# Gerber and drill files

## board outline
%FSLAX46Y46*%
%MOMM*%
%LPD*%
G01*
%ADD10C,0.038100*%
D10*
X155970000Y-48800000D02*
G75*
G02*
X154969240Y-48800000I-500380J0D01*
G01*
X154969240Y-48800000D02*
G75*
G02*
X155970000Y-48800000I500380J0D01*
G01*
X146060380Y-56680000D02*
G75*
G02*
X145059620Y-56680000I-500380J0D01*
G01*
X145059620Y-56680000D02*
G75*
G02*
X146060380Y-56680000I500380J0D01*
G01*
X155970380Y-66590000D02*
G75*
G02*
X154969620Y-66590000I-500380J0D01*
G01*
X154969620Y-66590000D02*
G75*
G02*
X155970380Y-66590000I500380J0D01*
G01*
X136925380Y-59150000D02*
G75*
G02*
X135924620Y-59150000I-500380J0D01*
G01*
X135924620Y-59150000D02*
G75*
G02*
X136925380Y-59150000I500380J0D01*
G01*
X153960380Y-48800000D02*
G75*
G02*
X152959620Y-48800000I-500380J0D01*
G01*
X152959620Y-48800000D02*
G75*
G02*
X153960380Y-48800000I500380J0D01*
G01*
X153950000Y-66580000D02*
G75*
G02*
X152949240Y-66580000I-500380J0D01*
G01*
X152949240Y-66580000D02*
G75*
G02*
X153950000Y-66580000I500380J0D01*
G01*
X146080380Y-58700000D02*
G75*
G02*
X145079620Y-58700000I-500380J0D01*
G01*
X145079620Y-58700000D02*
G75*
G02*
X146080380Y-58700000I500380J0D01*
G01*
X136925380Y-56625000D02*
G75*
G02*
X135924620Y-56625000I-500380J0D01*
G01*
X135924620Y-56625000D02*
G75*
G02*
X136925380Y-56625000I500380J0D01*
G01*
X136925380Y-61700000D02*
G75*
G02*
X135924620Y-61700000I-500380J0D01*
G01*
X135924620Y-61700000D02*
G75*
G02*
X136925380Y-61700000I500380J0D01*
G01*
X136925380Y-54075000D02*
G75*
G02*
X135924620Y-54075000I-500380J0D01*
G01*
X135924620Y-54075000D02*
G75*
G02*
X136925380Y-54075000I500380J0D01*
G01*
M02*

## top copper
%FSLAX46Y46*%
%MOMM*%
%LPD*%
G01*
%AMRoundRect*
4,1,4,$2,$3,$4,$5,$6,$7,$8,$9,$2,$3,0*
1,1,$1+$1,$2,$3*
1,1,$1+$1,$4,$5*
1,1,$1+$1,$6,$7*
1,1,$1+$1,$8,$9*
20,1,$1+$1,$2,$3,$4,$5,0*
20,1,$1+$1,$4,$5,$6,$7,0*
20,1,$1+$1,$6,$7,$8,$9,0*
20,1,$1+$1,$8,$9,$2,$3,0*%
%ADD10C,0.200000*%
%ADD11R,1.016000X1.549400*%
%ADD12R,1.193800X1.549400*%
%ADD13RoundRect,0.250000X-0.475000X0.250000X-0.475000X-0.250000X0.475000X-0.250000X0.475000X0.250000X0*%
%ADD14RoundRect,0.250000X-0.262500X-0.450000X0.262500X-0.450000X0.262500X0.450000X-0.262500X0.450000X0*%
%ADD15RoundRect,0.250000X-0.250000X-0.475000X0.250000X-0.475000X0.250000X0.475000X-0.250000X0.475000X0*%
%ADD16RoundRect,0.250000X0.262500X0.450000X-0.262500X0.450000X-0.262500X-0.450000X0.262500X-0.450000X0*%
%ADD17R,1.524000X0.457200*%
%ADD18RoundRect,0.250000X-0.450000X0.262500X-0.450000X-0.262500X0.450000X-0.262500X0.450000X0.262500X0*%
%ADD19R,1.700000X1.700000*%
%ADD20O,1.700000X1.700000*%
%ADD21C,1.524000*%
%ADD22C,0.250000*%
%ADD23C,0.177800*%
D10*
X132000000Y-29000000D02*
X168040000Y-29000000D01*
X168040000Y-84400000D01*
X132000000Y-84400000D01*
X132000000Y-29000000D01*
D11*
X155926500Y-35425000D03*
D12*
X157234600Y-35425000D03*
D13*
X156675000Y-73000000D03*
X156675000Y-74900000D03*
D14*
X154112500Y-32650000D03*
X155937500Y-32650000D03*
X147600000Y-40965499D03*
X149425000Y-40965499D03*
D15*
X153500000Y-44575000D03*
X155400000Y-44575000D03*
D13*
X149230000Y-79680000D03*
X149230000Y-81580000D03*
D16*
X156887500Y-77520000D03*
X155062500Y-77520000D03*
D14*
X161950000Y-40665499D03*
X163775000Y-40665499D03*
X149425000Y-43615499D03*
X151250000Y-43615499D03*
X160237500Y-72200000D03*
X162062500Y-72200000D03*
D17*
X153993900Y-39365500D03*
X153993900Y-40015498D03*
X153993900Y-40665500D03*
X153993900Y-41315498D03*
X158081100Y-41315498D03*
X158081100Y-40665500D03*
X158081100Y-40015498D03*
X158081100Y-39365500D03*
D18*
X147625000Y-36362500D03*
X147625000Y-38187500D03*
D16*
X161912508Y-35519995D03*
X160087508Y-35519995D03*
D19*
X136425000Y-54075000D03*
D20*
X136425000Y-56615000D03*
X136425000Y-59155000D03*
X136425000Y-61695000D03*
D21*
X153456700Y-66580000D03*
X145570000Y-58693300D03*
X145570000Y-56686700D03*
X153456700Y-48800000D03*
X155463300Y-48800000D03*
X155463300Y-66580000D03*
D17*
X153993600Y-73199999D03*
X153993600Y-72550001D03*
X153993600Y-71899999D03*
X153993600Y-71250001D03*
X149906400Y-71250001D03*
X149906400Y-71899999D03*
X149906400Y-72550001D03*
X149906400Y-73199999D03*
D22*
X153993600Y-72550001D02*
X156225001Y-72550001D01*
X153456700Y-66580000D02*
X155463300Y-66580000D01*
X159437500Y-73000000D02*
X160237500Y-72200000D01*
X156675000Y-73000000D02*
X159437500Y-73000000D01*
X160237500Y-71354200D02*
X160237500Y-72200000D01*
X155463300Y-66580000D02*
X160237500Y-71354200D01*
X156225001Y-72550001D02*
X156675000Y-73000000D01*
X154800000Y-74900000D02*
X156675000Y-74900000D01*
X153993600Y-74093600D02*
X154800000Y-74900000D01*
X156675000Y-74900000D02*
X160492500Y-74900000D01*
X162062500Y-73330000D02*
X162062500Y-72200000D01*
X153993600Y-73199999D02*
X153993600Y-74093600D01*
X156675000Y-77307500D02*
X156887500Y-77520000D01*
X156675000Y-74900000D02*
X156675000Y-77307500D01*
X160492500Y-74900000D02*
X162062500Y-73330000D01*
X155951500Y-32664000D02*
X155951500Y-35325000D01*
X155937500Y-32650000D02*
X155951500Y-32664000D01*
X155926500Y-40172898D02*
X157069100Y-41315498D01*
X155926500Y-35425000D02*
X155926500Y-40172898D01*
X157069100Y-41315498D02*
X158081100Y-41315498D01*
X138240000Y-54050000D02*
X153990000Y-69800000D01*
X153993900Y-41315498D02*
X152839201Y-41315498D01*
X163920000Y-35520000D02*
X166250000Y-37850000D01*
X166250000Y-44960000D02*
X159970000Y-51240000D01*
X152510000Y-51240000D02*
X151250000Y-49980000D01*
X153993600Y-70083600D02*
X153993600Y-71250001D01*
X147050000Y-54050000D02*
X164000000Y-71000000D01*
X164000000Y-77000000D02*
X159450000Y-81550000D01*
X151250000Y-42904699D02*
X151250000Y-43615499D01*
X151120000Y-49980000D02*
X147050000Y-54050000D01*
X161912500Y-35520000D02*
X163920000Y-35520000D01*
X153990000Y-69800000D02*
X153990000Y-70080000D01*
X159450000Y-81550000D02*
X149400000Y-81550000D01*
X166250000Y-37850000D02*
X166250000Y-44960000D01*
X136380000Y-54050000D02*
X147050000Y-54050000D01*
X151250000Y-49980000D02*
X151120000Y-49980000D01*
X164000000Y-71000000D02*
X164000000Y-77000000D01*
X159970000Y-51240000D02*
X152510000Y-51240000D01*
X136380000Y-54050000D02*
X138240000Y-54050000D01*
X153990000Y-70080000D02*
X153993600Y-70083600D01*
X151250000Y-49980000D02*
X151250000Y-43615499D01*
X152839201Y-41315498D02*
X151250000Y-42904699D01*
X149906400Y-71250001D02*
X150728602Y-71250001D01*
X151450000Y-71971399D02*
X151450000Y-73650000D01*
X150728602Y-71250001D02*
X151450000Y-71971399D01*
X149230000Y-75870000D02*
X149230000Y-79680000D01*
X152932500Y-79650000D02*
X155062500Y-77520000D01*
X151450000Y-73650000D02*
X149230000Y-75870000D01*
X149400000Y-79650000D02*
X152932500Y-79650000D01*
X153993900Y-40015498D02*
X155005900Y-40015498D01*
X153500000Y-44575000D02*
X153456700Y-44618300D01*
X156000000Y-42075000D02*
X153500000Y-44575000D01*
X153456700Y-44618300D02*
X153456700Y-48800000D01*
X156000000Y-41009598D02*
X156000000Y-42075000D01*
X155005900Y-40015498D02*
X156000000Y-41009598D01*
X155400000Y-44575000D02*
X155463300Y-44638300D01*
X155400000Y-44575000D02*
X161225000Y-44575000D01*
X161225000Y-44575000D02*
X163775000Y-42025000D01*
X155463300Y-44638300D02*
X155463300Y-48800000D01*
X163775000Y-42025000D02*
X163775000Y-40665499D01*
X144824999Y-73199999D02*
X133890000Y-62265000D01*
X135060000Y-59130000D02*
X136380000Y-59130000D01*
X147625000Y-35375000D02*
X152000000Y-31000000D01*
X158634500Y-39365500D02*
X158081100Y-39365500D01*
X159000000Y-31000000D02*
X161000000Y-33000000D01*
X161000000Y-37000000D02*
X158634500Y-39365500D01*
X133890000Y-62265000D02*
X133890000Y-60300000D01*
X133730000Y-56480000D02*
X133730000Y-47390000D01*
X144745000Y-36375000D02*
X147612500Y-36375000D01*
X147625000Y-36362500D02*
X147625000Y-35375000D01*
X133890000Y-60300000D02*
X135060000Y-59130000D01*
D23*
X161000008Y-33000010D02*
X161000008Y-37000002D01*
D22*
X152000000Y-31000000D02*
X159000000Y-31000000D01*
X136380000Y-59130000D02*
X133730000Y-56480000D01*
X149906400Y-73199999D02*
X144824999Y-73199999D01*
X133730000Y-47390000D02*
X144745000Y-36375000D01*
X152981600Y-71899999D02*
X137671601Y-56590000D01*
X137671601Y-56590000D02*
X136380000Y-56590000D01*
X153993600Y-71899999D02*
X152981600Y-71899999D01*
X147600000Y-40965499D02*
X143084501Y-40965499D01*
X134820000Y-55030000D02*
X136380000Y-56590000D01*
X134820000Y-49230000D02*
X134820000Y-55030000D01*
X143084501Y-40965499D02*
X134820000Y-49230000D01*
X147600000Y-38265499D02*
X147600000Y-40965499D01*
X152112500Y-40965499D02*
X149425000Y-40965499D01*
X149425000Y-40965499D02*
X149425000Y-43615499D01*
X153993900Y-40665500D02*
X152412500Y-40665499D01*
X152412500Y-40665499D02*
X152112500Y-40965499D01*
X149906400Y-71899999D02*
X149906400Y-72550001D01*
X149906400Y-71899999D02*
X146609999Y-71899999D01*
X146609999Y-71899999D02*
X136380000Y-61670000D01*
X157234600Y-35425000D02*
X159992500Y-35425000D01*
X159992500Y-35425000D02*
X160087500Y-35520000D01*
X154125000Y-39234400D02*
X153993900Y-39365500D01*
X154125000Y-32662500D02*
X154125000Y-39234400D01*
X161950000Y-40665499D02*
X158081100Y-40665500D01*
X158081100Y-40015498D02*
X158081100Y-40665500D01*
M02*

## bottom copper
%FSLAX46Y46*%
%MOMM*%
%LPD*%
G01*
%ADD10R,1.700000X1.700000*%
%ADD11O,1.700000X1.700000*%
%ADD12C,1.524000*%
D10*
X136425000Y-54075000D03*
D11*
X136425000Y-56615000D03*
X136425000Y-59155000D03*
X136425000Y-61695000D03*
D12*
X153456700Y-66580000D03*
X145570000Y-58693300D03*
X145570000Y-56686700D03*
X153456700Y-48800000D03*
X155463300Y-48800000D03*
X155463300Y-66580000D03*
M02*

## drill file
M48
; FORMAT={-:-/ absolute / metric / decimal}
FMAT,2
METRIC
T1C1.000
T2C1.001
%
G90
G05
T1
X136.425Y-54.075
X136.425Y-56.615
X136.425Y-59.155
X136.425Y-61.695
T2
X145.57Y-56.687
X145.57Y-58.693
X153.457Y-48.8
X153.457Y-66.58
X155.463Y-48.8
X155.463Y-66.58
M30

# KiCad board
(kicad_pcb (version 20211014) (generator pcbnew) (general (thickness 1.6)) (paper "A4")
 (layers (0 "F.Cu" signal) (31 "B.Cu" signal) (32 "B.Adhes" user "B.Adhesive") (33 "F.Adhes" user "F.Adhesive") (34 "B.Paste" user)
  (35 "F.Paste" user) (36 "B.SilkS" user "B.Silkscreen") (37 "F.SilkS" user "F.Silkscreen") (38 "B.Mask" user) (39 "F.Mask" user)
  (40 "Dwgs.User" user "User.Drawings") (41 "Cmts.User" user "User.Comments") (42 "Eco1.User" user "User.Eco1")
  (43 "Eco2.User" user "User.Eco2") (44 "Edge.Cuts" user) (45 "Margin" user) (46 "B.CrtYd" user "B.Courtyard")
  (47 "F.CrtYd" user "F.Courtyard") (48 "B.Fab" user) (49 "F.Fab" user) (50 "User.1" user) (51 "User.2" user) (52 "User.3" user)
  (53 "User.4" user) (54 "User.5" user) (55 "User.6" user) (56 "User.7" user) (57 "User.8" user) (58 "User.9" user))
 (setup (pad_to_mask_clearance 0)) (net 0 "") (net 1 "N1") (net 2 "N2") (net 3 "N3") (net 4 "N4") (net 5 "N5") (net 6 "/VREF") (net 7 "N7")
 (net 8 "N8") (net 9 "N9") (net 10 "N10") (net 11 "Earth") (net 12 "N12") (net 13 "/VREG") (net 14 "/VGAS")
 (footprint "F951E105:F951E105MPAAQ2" (layer "F.Cu") (at 156.625 35.425)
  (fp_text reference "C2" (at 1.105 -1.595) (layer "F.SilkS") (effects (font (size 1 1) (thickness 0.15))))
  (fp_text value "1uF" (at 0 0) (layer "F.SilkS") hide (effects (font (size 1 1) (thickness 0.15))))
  (pad "1" smd rect (at -0.6985 0) (size 1.016 1.5494) (layers "F.Cu" "F.Paste" "F.Mask") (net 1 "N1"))
  (pad "2" smd rect (at 0.6096 0) (size 1.1938 1.5494) (layers "F.Cu" "F.Paste" "F.Mask") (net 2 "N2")))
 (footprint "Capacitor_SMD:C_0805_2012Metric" (layer "F.Cu") (at 156.675 73.95 -90)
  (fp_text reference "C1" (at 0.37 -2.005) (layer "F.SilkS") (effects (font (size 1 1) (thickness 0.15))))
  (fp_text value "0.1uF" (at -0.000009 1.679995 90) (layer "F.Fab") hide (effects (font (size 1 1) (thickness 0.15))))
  (pad "1" smd roundrect (at -0.95 0 270) (size 1 1.45) (layers "F.Cu" "F.Paste" "F.Mask") (roundrect_rratio 0.25) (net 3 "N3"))
  (pad "2" smd roundrect (at 0.95 0 270) (size 1 1.45) (layers "F.Cu" "F.Paste" "F.Mask") (roundrect_rratio 0.25) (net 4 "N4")))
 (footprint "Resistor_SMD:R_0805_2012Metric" (layer "F.Cu") (at 155.025 32.65)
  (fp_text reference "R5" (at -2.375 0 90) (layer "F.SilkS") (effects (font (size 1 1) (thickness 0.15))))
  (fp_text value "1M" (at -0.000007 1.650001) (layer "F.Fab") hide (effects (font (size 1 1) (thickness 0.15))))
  (pad "1" smd roundrect (at -0.9125 0) (size 1.025 1.4) (layers "F.Cu" "F.Paste" "F.Mask") (roundrect_rratio 0.243902439) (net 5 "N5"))
  (pad "2" smd roundrect (at 0.9125 0) (size 1.025 1.4) (layers "F.Cu" "F.Paste" "F.Mask") (roundrect_rratio 0.243902439) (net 1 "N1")))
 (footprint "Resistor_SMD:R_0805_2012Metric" (layer "F.Cu") (at 148.5125 40.965499)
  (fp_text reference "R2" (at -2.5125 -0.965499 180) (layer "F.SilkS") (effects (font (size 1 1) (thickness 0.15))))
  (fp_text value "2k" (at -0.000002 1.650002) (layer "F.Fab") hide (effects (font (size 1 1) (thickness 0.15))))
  (pad "1" smd roundrect (at -0.9125 0) (size 1.025 1.4) (layers "F.Cu" "F.Paste" "F.Mask") (roundrect_rratio 0.243902439) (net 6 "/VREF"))
  (pad "2" smd roundrect (at 0.9125 0) (size 1.025 1.4) (layers "F.Cu" "F.Paste" "F.Mask") (roundrect_rratio 0.243902439) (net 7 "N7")))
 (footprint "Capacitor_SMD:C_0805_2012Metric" (layer "F.Cu") (at 154.45 44.575)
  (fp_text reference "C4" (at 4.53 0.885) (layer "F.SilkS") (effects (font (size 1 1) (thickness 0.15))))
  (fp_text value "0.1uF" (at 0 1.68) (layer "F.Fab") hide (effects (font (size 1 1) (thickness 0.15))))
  (pad "1" smd roundrect (at -0.95 0) (size 1 1.45) (layers "F.Cu" "F.Paste" "F.Mask") (roundrect_rratio 0.25) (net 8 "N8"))
  (pad "2" smd roundrect (at 0.95 0) (size 1 1.45) (layers "F.Cu" "F.Paste" "F.Mask") (roundrect_rratio 0.25) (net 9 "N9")))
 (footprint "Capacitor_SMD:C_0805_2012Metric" (layer "F.Cu") (at 149.23 80.63 -90)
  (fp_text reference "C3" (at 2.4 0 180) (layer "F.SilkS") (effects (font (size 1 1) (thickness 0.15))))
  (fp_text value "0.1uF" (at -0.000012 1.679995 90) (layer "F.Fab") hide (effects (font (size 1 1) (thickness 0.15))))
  (pad "1" smd roundrect (at -0.95 0 270) (size 1 1.45) (layers "F.Cu" "F.Paste" "F.Mask") (roundrect_rratio 0.25) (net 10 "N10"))
  (pad "2" smd roundrect (at 0.95 0 270) (size 1 1.45) (layers "F.Cu" "F.Paste" "F.Mask") (roundrect_rratio 0.25) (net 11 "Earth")))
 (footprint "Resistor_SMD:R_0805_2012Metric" (layer "F.Cu") (at 155.975 77.52 180)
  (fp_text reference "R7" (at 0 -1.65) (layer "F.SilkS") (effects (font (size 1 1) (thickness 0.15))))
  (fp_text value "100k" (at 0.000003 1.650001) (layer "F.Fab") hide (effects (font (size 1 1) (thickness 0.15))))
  (pad "1" smd roundrect (at -0.9125 0 180) (size 1.025 1.4) (layers "F.Cu" "F.Paste" "F.Mask") (roundrect_rratio 0.243902439) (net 4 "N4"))
  (pad "2" smd roundrect (at 0.9125 0 180) (size 1.025 1.4) (layers "F.Cu" "F.Paste" "F.Mask") (roundrect_rratio 0.243902439) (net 10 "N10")))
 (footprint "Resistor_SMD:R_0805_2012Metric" (layer "F.Cu") (at 162.8625 40.665499)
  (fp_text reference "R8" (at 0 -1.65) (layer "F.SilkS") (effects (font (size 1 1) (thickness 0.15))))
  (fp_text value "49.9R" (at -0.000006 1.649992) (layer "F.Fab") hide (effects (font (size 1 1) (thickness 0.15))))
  (pad "1" smd roundrect (at -0.9125 0) (size 1.025 1.4) (layers "F.Cu" "F.Paste" "F.Mask") (roundrect_rratio 0.243902439) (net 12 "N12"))
  (pad "2" smd roundrect (at 0.9125 0) (size 1.025 1.4) (layers "F.Cu" "F.Paste" "F.Mask") (roundrect_rratio 0.243902439) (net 9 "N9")))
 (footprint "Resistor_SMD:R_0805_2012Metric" (layer "F.Cu") (at 150.3375 43.615499)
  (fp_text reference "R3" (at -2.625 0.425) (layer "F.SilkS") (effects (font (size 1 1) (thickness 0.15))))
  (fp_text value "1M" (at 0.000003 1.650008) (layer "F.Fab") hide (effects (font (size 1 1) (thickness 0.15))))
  (pad "1" smd roundrect (at -0.9125 0) (size 1.025 1.4) (layers "F.Cu" "F.Paste" "F.Mask") (roundrect_rratio 0.243902439) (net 7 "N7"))
  (pad "2" smd roundrect (at 0.9125 0) (size 1.025 1.4) (layers "F.Cu" "F.Paste" "F.Mask") (roundrect_rratio 0.243902439) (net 11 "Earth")))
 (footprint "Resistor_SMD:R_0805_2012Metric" (layer "F.Cu") (at 161.15 72.2)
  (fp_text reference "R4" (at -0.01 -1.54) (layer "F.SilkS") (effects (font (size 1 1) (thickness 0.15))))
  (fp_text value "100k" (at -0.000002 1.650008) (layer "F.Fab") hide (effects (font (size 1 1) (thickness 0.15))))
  (pad "1" smd roundrect (at -0.9125 0) (size 1.025 1.4) (layers "F.Cu" "F.Paste" "F.Mask") (roundrect_rratio 0.243902439) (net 3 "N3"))
  (pad "2" smd roundrect (at 0.9125 0) (size 1.025 1.4) (layers "F.Cu" "F.Paste" "F.Mask") (roundrect_rratio 0.243902439) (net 4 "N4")))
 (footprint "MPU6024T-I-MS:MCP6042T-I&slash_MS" (layer "F.Cu") (at 156.0375 40.340499)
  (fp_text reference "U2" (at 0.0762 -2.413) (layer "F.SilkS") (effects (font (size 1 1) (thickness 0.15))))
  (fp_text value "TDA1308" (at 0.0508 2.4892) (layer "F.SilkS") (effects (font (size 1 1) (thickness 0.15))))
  (pad "1" smd rect (at -2.0436 -0.974999) (size 1.524 0.4572) (layers "F.Cu" "F.Paste" "F.Mask") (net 5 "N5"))
  (pad "2" smd rect (at -2.0436 -0.325001) (size 1.524 0.4572) (layers "F.Cu" "F.Paste" "F.Mask") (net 8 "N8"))
  (pad "3" smd rect (at -2.0436 0.325001) (size 1.524 0.4572) (layers "F.Cu" "F.Paste" "F.Mask") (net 7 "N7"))
  (pad "4" smd rect (at -2.0436 0.974999) (size 1.524 0.4572) (layers "F.Cu" "F.Paste" "F.Mask") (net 11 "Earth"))
  (pad "5" smd rect (at 2.0436 0.974999) (size 1.524 0.4572) (layers "F.Cu" "F.Paste" "F.Mask") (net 1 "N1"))
  (pad "6" smd rect (at 2.0436 0.325001) (size 1.524 0.4572) (layers "F.Cu" "F.Paste" "F.Mask") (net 12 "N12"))
  (pad "7" smd rect (at 2.0436 -0.325001) (size 1.524 0.4572) (layers "F.Cu" "F.Paste" "F.Mask") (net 12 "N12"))
  (pad "8" smd rect (at 2.0436 -0.974999) (size 1.524 0.4572) (layers "F.Cu" "F.Paste" "F.Mask") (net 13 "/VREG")))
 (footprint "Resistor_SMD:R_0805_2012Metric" (layer "F.Cu") (at 147.625 37.275 -90)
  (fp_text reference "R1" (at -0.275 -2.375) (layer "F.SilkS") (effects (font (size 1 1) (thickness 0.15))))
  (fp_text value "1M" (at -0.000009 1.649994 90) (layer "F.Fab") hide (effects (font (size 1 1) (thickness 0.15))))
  (pad "1" smd roundrect (at -0.9125 0 270) (size 1.025 1.4) (layers "F.Cu" "F.Paste" "F.Mask") (roundrect_rratio 0.243902439)
   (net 13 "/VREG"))
  (pad "2" smd roundrect (at 0.9125 0 270) (size 1.025 1.4) (layers "F.Cu" "F.Paste" "F.Mask") (roundrect_rratio 0.243902439)
   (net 6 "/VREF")))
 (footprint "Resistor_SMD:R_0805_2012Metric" (layer "F.Cu") (at 161.000008 35.519995 180)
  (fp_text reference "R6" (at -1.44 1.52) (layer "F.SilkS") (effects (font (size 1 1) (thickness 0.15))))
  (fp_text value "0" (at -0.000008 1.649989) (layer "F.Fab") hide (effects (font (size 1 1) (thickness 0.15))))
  (pad "1" smd roundrect (at -0.9125 0 180) (size 1.025 1.4) (layers "F.Cu" "F.Paste" "F.Mask") (roundrect_rratio 0.243902439)
   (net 11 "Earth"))
  (pad "2" smd roundrect (at 0.9125 0 180) (size 1.025 1.4) (layers "F.Cu" "F.Paste" "F.Mask") (roundrect_rratio 0.243902439) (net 2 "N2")))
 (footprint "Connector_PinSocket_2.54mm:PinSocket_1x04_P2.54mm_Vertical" (layer "F.Cu") (at 136.425 54.075)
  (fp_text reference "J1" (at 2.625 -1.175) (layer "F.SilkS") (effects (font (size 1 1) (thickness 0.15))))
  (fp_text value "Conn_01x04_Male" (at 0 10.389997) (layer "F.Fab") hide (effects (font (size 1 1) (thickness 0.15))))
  (pad "1" thru_hole rect (at 0 0) (size 1.7 1.7) (drill 1) (layers *.Cu *.Mask) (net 11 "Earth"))
  (pad "2" thru_hole oval (at 0 2.54) (size 1.7 1.7) (drill 1) (layers *.Cu *.Mask) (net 6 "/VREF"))
  (pad "3" thru_hole oval (at 0 5.08) (size 1.7 1.7) (drill 1) (layers *.Cu *.Mask) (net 13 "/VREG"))
  (pad "4" thru_hole oval (at 0 7.62) (size 1.7 1.7) (drill 1) (layers *.Cu *.Mask) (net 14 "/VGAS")))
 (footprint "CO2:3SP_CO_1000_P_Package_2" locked (layer "F.Cu") (at 154.46 57.69)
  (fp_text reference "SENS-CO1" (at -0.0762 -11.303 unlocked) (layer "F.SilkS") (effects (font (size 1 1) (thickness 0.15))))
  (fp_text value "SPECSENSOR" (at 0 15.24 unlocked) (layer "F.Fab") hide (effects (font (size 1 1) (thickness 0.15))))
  (pad "1" thru_hole circle locked (at -1.0033 8.89) (size 1.524 1.524) (drill 1.00076) (layers *.Cu *.Mask) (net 3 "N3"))
  (pad "2" thru_hole circle locked (at -8.89 1.0033) (size 1.524 1.524) (drill 1.00076) (layers *.Cu *.Mask))
  (pad "3" thru_hole circle locked (at -8.89 -1.0033) (size 1.524 1.524) (drill 1.00076) (layers *.Cu *.Mask))
  (pad "4" thru_hole circle locked (at -1.0033 -8.89) (size 1.524 1.524) (drill 1.00076) (layers *.Cu *.Mask) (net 8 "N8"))
  (pad "5" thru_hole circle locked (at 1.0033 -8.89) (size 1.524 1.524) (drill 1.00076) (layers *.Cu *.Mask) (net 9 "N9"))
  (pad "6" thru_hole circle locked (at 1.0033 8.89) (size 1.524 1.524) (drill 1.00076) (layers *.Cu "F.Mask") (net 3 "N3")))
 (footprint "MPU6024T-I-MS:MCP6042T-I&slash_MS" (layer "F.Cu") (at 151.95 72.225 180)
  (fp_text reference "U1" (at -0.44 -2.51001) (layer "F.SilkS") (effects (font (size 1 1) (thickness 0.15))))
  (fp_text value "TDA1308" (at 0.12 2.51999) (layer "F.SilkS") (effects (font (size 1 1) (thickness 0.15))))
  (pad "1" smd rect (at -2.0436 -0.974999 180) (size 1.524 0.4572) (layers "F.Cu" "F.Paste" "F.Mask") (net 4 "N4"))
  (pad "2" smd rect (at -2.0436 -0.325001 180) (size 1.524 0.4572) (layers "F.Cu" "F.Paste" "F.Mask") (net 3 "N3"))
  (pad "3" smd rect (at -2.0436 0.325001 180) (size 1.524 0.4572) (layers "F.Cu" "F.Paste" "F.Mask") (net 6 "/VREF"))
  (pad "4" smd rect (at -2.0436 0.974999 180) (size 1.524 0.4572) (layers "F.Cu" "F.Paste" "F.Mask") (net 11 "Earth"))
  (pad "5" smd rect (at 2.0436 0.974999 180) (size 1.524 0.4572) (layers "F.Cu" "F.Paste" "F.Mask") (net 10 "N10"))
  (pad "6" smd rect (at 2.0436 0.325001 180) (size 1.524 0.4572) (layers "F.Cu" "F.Paste" "F.Mask") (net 14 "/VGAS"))
  (pad "7" smd rect (at 2.0436 -0.325001 180) (size 1.524 0.4572) (layers "F.Cu" "F.Paste" "F.Mask") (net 14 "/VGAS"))
  (pad "8" smd rect (at 2.0436 -0.974999 180) (size 1.524 0.4572) (layers "F.Cu" "F.Paste" "F.Mask") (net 13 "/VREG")))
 (gr_rect (start 132 29) (end 168.04 84.4) (layer "F.Cu") (width 0.2) (fill none))
 (gr_circle (center 155.46962 48.8) (end 155.97 48.8) (layer "Edge.Cuts") (width 0.0381) (fill none))
 (gr_circle (center 145.56 56.68) (end 146.06038 56.68) (layer "Edge.Cuts") (width 0.0381) (fill none))
 (gr_circle (center 155.47 66.59) (end 155.97038 66.59) (layer "Edge.Cuts") (width 0.0381) (fill none))
 (gr_circle (center 136.425 59.15) (end 136.92538 59.15) (layer "Edge.Cuts") (width 0.0381) (fill none))
 (gr_circle (center 153.46 48.8) (end 153.96038 48.8) (layer "Edge.Cuts") (width 0.0381) (fill none))
 (gr_circle (center 153.44962 66.58) (end 153.95 66.58) (layer "Edge.Cuts") (width 0.0381) (fill none))
 (gr_circle (center 145.58 58.7) (end 146.08038 58.7) (layer "Edge.Cuts") (width 0.0381) (fill none))
 (gr_circle (center 136.425 56.625) (end 136.92538 56.625) (layer "Edge.Cuts") (width 0.0381) (fill none))
 (gr_circle (center 136.425 61.7) (end 136.92538 61.7) (layer "Edge.Cuts") (width 0.0381) (fill none))
 (gr_circle (center 136.425 54.075) (end 136.92538 54.075) (layer "Edge.Cuts") (width 0.0381) (fill none))
 (segment (start 153.9936 72.550001) (end 156.225001 72.550001) (width 0.25) (layer "F.Cu") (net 3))
 (segment (start 153.4567 66.58) (end 155.4633 66.58) (width 0.25) (layer "F.Cu") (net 3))
 (segment (start 159.4375 73) (end 160.2375 72.2) (width 0.25) (layer "F.Cu") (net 3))
 (segment (start 156.675 73) (end 159.4375 73) (width 0.25) (layer "F.Cu") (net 3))
 (segment (start 160.2375 71.3542) (end 160.2375 72.2) (width 0.25) (layer "F.Cu") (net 3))
 (segment (start 155.4633 66.58) (end 160.2375 71.3542) (width 0.25) (layer "F.Cu") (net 3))
 (segment (start 156.225001 72.550001) (end 156.675 73) (width 0.25) (layer "F.Cu") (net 3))
 (segment (start 154.8 74.9) (end 156.675 74.9) (width 0.25) (layer "F.Cu") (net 4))
 (segment (start 153.9936 74.0936) (end 154.8 74.9) (width 0.25) (layer "F.Cu") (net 4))
 (segment (start 156.675 74.9) (end 160.4925 74.9) (width 0.25) (layer "F.Cu") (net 4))
 (segment (start 162.0625 73.33) (end 162.0625 72.2) (width 0.25) (layer "F.Cu") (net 4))
 (segment (start 153.9936 73.199999) (end 153.9936 74.0936) (width 0.25) (layer "F.Cu") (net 4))
 (segment (start 156.675 77.3075) (end 156.8875 77.52) (width 0.25) (layer "F.Cu") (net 4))
 (segment (start 156.675 74.9) (end 156.675 77.3075) (width 0.25) (layer "F.Cu") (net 4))
 (segment (start 160.4925 74.9) (end 162.0625 73.33) (width 0.25) (layer "F.Cu") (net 4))
 (segment (start 155.9515 32.664) (end 155.9515 35.325) (width 0.25) (layer "F.Cu") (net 1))
 (segment (start 155.9375 32.65) (end 155.9515 32.664) (width 0.25) (layer "F.Cu") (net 1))
 (segment (start 155.9265 40.172898) (end 157.0691 41.315498) (width 0.25) (layer "F.Cu") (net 1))
 (segment (start 155.9265 35.425) (end 155.9265 40.172898) (width 0.25) (layer "F.Cu") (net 1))
 (segment (start 157.0691 41.315498) (end 158.0811 41.315498) (width 0.25) (layer "F.Cu") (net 1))
 (segment (start 138.24 54.05) (end 153.99 69.8) (width 0.25) (layer "F.Cu") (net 11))
 (segment (start 153.9939 41.315498) (end 152.839201 41.315498) (width 0.25) (layer "F.Cu") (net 11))
 (segment (start 163.92 35.52) (end 166.25 37.85) (width 0.25) (layer "F.Cu") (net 11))
 (segment (start 166.25 44.96) (end 159.97 51.24) (width 0.25) (layer "F.Cu") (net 11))
 (segment (start 152.51 51.24) (end 151.25 49.98) (width 0.25) (layer "F.Cu") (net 11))
 (segment (start 153.9936 70.0836) (end 153.9936 71.250001) (width 0.25) (layer "F.Cu") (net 11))
 (segment (start 147.05 54.05) (end 164 71) (width 0.25) (layer "F.Cu") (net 11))
 (segment (start 164 77) (end 159.45 81.55) (width 0.25) (layer "F.Cu") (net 11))
 (segment (start 151.25 42.904699) (end 151.25 43.615499) (width 0.25) (layer "F.Cu") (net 11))
 (segment (start 151.12 49.98) (end 147.05 54.05) (width 0.25) (layer "F.Cu") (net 11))
 (segment (start 161.9125 35.52) (end 163.92 35.52) (width 0.25) (layer "F.Cu") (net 11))
 (segment (start 153.99 69.8) (end 153.99 70.08) (width 0.25) (layer "F.Cu") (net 11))
 (segment (start 159.45 81.55) (end 149.4 81.55) (width 0.25) (layer "F.Cu") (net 11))
 (segment (start 166.25 37.85) (end 166.25 44.96) (width 0.25) (layer "F.Cu") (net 11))
 (segment (start 136.38 54.05) (end 147.05 54.05) (width 0.25) (layer "F.Cu") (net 11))
 (segment (start 151.25 49.98) (end 151.12 49.98) (width 0.25) (layer "F.Cu") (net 11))
 (segment (start 164 71) (end 164 77) (width 0.25) (layer "F.Cu") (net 11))
 (segment (start 159.97 51.24) (end 152.51 51.24) (width 0.25) (layer "F.Cu") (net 11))
 (segment (start 136.38 54.05) (end 138.24 54.05) (width 0.25) (layer "F.Cu") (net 11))
 (segment (start 153.99 70.08) (end 153.9936 70.0836) (width 0.25) (layer "F.Cu") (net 11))
 (segment (start 151.25 49.98) (end 151.25 43.615499) (width 0.25) (layer "F.Cu") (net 11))
 (segment (start 152.839201 41.315498) (end 151.25 42.904699) (width 0.25) (layer "F.Cu") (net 11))
 (segment (start 149.9064 71.250001) (end 150.728602 71.250001) (width 0.25) (layer "F.Cu") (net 10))
 (segment (start 151.45 71.971399) (end 151.45 73.65) (width 0.25) (layer "F.Cu") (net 10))
 (segment (start 150.728602 71.250001) (end 151.45 71.971399) (width 0.25) (layer "F.Cu") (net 10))
 (segment (start 149.23 75.87) (end 149.23 79.68) (width 0.25) (layer "F.Cu") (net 10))
 (segment (start 152.9325 79.65) (end 155.0625 77.52) (width 0.25) (layer "F.Cu") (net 10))
 (segment (start 151.45 73.65) (end 149.23 75.87) (width 0.25) (layer "F.Cu") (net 10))
 (segment (start 149.4 79.65) (end 152.9325 79.65) (width 0.25) (layer "F.Cu") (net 10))
 (segment (start 153.9939 40.015498) (end 155.0059 40.015498) (width 0.25) (layer "F.Cu") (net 8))
 (segment (start 153.5 44.575) (end 153.4567 44.6183) (width 0.25) (layer "F.Cu") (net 8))
 (segment (start 156 42.075) (end 153.5 44.575) (width 0.25) (layer "F.Cu") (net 8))
 (segment (start 153.4567 44.6183) (end 153.4567 48.8) (width 0.25) (layer "F.Cu") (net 8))
 (segment (start 156 41.009598) (end 156 42.075) (width 0.25) (layer "F.Cu") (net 8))
 (segment (start 155.0059 40.015498) (end 156 41.009598) (width 0.25) (layer "F.Cu") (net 8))
 (segment (start 155.4 44.575) (end 155.4633 44.6383) (width 0.25) (layer "F.Cu") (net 9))
 (segment (start 155.4 44.575) (end 161.225 44.575) (width 0.25) (layer "F.Cu") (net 9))
 (segment (start 161.225 44.575) (end 163.775 42.025) (width 0.25) (layer "F.Cu") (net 9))
 (segment (start 155.4633 44.6383) (end 155.4633 48.8) (width 0.25) (layer "F.Cu") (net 9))
 (segment (start 163.775 42.025) (end 163.775 40.665499) (width 0.25) (layer "F.Cu") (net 9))
 (segment (start 144.824999 73.199999) (end 133.89 62.265) (width 0.25) (layer "F.Cu") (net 13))
 (segment (start 135.06 59.13) (end 136.38 59.13) (width 0.25) (layer "F.Cu") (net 13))
 (segment (start 147.625 35.375) (end 152 31) (width 0.25) (layer "F.Cu") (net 13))
 (segment (start 158.6345 39.3655) (end 158.0811 39.3655) (width 0.25) (layer "F.Cu") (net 13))
 (segment (start 159 31) (end 161 33) (width 0.25) (layer "F.Cu") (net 13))
 (segment (start 161 37) (end 158.6345 39.3655) (width 0.25) (layer "F.Cu") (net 13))
 (segment (start 133.89 62.265) (end 133.89 60.3) (width 0.25) (layer "F.Cu") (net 13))
 (segment (start 133.73 56.48) (end 133.73 47.39) (width 0.25) (layer "F.Cu") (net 13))
 (segment (start 144.745 36.375) (end 147.6125 36.375) (width 0.25) (layer "F.Cu") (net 13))
 (segment (start 147.625 36.3625) (end 147.625 35.375) (width 0.25) (layer "F.Cu") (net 13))
 (segment (start 133.89 60.3) (end 135.06 59.13) (width 0.25) (layer "F.Cu") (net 13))
 (segment (start 161.000008 33.00001) (end 161.000008 37.000002) (width 0.1778) (layer "F.Cu") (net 13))
 (segment (start 152 31) (end 159 31) (width 0.25) (layer "F.Cu") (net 13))
 (segment (start 136.38 59.13) (end 133.73 56.48) (width 0.25) (layer "F.Cu") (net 13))
 (segment (start 149.9064 73.199999) (end 144.824999 73.199999) (width 0.25) (layer "F.Cu") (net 13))
 (segment (start 133.73 47.39) (end 144.745 36.375) (width 0.25) (layer "F.Cu") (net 13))
 (segment (start 152.9816 71.899999) (end 137.671601 56.59) (width 0.25) (layer "F.Cu") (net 6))
 (segment (start 137.671601 56.59) (end 136.38 56.59) (width 0.25) (layer "F.Cu") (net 6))
 (segment (start 153.9936 71.899999) (end 152.9816 71.899999) (width 0.25) (layer "F.Cu") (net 6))
 (segment (start 147.6 40.965499) (end 143.084501 40.965499) (width 0.25) (layer "F.Cu") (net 6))
 (segment (start 134.82 55.03) (end 136.38 56.59) (width 0.25) (layer "F.Cu") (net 6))
 (segment (start 134.82 49.23) (end 134.82 55.03) (width 0.25) (layer "F.Cu") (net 6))
 (segment (start 143.084501 40.965499) (end 134.82 49.23) (width 0.25) (layer "F.Cu") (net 6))
 (segment (start 147.6 38.265499) (end 147.6 40.965499) (width 0.25) (layer "F.Cu") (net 6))
 (segment (start 152.1125 40.965499) (end 149.425 40.965499) (width 0.25) (layer "F.Cu") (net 7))
 (segment (start 149.425 40.965499) (end 149.425 43.615499) (width 0.25) (layer "F.Cu") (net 7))
 (segment (start 153.9939 40.6655) (end 152.4125 40.665499) (width 0.25) (layer "F.Cu") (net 7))
 (segment (start 152.4125 40.665499) (end 152.1125 40.965499) (width 0.25) (layer "F.Cu") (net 7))
 (segment (start 149.9064 71.899999) (end 149.9064 72.550001) (width 0.25) (layer "F.Cu") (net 14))
 (segment (start 149.9064 71.899999) (end 146.609999 71.899999) (width 0.25) (layer "F.Cu") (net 14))
 (segment (start 146.609999 71.899999) (end 136.38 61.67) (width 0.25) (layer "F.Cu") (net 14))
 (segment (start 157.2346 35.425) (end 159.9925 35.425) (width 0.25) (layer "F.Cu") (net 2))
 (segment (start 159.9925 35.425) (end 160.0875 35.52) (width 0.25) (layer "F.Cu") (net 2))
 (segment (start 154.125 39.2344) (end 153.9939 39.3655) (width 0.25) (layer "F.Cu") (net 5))
 (segment (start 154.125 32.6625) (end 154.125 39.2344) (width 0.25) (layer "F.Cu") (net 5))
 (segment (start 161.95 40.665499) (end 158.0811 40.6655) (width 0.25) (layer "F.Cu") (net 12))
 (segment (start 158.0811 40.015498) (end 158.0811 40.6655) (width 0.25) (layer "F.Cu") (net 12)))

